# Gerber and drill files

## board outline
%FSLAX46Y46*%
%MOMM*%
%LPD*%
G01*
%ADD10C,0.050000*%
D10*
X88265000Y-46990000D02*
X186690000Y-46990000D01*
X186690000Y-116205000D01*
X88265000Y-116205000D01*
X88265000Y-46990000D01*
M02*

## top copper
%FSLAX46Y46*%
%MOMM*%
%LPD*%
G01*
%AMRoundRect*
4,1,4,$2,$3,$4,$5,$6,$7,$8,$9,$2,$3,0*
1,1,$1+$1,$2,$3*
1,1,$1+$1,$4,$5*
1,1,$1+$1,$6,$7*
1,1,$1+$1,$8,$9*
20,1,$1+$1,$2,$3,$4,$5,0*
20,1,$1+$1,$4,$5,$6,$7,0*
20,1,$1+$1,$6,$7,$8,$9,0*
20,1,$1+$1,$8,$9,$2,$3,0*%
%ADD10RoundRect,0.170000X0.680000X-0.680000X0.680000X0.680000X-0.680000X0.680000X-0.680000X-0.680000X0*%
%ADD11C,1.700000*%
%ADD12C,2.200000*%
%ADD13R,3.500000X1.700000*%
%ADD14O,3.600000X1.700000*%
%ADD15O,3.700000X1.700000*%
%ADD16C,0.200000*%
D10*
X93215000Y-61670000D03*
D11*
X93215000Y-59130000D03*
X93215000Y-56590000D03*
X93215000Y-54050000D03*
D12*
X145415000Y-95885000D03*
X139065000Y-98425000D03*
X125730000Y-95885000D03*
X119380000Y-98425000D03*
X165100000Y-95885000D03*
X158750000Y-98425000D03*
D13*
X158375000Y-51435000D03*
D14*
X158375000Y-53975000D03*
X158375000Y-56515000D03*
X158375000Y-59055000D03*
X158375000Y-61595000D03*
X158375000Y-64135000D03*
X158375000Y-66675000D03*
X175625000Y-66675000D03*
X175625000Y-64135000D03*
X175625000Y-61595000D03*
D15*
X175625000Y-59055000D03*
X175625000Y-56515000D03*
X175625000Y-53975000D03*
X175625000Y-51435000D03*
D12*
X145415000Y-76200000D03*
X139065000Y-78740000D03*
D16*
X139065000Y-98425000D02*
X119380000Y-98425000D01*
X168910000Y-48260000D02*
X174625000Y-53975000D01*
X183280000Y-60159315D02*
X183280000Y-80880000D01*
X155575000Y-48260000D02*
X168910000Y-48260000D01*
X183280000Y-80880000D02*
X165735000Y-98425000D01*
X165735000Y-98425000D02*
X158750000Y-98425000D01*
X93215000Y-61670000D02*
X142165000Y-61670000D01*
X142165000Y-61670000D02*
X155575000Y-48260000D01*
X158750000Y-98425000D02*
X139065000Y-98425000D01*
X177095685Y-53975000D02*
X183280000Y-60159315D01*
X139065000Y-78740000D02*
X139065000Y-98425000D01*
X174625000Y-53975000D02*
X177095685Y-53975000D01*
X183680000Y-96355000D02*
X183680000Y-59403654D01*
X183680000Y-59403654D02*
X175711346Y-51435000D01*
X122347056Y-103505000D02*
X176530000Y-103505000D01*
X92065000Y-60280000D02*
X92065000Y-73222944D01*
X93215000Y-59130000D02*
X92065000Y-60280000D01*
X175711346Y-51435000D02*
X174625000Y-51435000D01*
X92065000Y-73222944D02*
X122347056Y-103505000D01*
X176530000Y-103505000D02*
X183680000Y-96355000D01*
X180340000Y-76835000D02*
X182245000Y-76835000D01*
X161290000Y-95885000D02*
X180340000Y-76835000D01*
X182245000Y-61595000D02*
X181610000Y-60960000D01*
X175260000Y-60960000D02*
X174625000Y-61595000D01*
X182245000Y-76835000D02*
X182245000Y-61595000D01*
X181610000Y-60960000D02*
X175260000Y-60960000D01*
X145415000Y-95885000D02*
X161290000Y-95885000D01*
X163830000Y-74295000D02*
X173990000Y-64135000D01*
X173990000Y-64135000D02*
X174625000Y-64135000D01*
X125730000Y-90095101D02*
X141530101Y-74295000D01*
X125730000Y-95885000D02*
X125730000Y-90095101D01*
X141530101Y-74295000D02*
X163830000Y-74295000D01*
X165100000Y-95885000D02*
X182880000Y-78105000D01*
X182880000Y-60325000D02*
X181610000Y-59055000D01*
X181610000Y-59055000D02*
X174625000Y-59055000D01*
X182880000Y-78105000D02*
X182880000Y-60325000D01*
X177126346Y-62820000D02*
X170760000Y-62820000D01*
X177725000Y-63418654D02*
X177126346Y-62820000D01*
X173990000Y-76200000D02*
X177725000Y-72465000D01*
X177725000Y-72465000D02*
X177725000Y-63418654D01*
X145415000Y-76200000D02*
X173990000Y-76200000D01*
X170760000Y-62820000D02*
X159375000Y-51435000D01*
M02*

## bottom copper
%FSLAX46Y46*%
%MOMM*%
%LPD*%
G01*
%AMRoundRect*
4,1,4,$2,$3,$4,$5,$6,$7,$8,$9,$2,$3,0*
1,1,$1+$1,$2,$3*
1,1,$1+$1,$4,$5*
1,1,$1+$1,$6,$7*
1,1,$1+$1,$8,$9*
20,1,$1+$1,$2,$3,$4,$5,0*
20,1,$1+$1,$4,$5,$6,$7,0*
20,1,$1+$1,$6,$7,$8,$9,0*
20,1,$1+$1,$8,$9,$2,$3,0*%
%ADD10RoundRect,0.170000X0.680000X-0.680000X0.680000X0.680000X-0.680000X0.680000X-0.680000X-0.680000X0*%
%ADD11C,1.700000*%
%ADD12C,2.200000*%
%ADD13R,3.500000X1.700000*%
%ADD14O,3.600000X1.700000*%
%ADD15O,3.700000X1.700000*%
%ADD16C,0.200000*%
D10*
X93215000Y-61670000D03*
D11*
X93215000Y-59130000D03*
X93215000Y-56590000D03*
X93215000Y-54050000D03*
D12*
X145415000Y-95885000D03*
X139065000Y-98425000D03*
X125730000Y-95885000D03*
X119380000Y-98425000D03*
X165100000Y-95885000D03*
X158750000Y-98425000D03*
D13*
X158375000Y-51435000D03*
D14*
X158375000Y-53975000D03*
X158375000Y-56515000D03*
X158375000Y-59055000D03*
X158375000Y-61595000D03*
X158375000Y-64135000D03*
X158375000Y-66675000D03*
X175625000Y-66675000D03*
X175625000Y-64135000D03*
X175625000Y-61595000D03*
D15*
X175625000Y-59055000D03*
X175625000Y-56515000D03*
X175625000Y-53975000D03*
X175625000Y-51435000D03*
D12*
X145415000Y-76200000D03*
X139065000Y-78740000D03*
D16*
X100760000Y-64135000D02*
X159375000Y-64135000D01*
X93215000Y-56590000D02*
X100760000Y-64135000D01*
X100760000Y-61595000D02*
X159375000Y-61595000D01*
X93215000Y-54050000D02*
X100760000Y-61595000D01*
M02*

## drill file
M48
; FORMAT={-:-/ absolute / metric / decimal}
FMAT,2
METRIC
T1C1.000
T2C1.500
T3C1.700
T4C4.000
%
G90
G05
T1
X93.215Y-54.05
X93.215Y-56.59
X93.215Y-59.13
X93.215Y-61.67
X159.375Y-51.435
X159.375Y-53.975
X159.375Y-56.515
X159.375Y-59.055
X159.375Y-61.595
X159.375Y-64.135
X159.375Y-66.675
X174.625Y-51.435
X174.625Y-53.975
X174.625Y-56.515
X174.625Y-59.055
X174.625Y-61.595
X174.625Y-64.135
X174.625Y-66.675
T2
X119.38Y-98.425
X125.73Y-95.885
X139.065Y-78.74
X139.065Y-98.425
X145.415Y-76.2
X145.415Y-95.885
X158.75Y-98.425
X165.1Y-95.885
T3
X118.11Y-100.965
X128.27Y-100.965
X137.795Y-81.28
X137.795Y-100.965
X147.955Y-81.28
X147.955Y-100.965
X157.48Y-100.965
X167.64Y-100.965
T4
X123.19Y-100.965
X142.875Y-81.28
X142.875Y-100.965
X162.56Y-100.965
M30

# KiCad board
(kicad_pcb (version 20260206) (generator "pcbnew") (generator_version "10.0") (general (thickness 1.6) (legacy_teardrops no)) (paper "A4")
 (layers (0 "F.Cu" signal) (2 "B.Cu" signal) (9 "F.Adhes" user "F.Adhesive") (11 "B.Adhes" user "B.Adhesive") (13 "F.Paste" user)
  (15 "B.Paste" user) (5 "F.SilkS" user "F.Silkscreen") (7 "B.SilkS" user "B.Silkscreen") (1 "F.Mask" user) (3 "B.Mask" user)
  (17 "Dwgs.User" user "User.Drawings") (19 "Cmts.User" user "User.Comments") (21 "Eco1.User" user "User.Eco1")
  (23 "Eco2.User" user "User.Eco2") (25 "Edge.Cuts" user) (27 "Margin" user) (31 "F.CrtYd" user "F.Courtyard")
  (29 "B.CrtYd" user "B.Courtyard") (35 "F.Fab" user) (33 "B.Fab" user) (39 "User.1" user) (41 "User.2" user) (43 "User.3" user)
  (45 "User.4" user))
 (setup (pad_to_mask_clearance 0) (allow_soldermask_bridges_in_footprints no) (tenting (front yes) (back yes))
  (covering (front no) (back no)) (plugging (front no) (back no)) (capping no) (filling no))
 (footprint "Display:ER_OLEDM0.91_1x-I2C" (layer "F.Cu") (at 93.215 61.67 90)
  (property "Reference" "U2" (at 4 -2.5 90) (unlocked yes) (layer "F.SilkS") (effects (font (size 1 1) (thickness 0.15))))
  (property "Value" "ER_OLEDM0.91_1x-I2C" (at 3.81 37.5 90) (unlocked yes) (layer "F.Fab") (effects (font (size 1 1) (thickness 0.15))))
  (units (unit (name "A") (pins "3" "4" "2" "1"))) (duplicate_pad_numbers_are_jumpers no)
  (pad "1" thru_hole roundrect (at 0 0 90) (size 1.7 1.7) (drill 1) (layers "*.Cu" "*.Mask") (remove_unused_layers no)
   (roundrect_rratio 0.1) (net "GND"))
  (pad "2" thru_hole circle (at 2.54 0 90) (size 1.7 1.7) (drill 1) (layers "*.Cu" "*.Mask") (remove_unused_layers no) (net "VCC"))
  (pad "3" thru_hole circle (at 5.08 0 90) (size 1.7 1.7) (drill 1) (layers "*.Cu" "*.Mask") (remove_unused_layers no)
   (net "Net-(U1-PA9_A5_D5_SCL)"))
  (pad "4" thru_hole circle (at 7.62 0 90) (size 1.7 1.7) (drill 1) (layers "*.Cu" "*.Mask") (remove_unused_layers no)
   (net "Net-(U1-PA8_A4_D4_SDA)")))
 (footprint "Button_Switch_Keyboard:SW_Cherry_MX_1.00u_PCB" (layer "F.Cu") (at 145.415 95.885)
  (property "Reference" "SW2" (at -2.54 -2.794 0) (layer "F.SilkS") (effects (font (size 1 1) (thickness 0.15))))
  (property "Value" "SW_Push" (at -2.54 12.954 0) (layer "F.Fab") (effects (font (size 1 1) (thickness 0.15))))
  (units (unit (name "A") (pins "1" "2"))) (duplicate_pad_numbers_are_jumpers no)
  (pad "" np_thru_hole circle (at -7.62 5.08) (size 1.7 1.7) (drill 1.7) (layers "*.Cu" "*.Mask"))
  (pad "" np_thru_hole circle (at -2.54 5.08) (size 4 4) (drill 4) (layers "*.Cu" "*.Mask"))
  (pad "" np_thru_hole circle (at 2.54 5.08) (size 1.7 1.7) (drill 1.7) (layers "*.Cu" "*.Mask"))
  (pad "1" thru_hole circle (at 0 0) (size 2.2 2.2) (drill 1.5) (layers "*.Cu" "*.Mask") (remove_unused_layers no)
   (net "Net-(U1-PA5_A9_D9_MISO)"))
  (pad "2" thru_hole circle (at -6.35 2.54) (size 2.2 2.2) (drill 1.5) (layers "*.Cu" "*.Mask") (remove_unused_layers no) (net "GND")))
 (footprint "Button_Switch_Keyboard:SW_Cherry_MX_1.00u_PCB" (layer "F.Cu") (at 125.73 95.885)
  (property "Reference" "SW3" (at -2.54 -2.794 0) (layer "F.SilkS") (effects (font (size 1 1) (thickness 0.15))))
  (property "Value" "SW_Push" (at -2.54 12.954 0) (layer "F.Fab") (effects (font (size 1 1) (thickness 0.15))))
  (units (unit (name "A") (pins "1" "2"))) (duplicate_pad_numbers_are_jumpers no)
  (pad "" np_thru_hole circle (at -7.62 5.08) (size 1.7 1.7) (drill 1.7) (layers "*.Cu" "*.Mask"))
  (pad "" np_thru_hole circle (at -2.54 5.08) (size 4 4) (drill 4) (layers "*.Cu" "*.Mask"))
  (pad "" np_thru_hole circle (at 2.54 5.08) (size 1.7 1.7) (drill 1.7) (layers "*.Cu" "*.Mask"))
  (pad "1" thru_hole circle (at 0 0) (size 2.2 2.2) (drill 1.5) (layers "*.Cu" "*.Mask") (remove_unused_layers no)
   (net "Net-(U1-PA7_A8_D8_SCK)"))
  (pad "2" thru_hole circle (at -6.35 2.54) (size 2.2 2.2) (drill 1.5) (layers "*.Cu" "*.Mask") (remove_unused_layers no) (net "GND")))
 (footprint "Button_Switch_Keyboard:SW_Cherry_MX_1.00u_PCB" (layer "F.Cu") (at 165.1 95.885)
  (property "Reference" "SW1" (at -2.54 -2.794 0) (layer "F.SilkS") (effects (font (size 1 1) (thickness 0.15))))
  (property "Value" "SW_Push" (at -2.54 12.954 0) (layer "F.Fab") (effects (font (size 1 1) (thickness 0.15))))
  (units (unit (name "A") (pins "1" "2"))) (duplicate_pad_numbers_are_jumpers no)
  (pad "" np_thru_hole circle (at -7.62 5.08) (size 1.7 1.7) (drill 1.7) (layers "*.Cu" "*.Mask"))
  (pad "" np_thru_hole circle (at -2.54 5.08) (size 4 4) (drill 4) (layers "*.Cu" "*.Mask"))
  (pad "" np_thru_hole circle (at 2.54 5.08) (size 1.7 1.7) (drill 1.7) (layers "*.Cu" "*.Mask"))
  (pad "1" thru_hole circle (at 0 0) (size 2.2 2.2) (drill 1.5) (layers "*.Cu" "*.Mask") (remove_unused_layers no)
   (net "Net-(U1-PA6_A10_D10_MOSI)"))
  (pad "2" thru_hole circle (at -6.35 2.54) (size 2.2 2.2) (drill 1.5) (layers "*.Cu" "*.Mask") (remove_unused_layers no) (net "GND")))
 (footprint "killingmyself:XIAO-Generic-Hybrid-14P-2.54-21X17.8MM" (layer "F.Cu") (at 167 59.055)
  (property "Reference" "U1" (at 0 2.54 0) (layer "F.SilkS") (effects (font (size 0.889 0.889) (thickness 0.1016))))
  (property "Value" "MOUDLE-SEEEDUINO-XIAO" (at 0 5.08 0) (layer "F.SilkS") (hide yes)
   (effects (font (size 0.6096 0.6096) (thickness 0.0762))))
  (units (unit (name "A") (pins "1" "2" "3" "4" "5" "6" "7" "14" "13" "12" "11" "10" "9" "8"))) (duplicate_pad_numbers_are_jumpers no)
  (pad "1" thru_hole rect (at -7.625 -7.62) (size 3.5 1.7) (drill 1 (offset -1 0)) (layers "*.Cu" "*.Mask") (remove_unused_layers no)
   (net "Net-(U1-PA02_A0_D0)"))
  (pad "2" thru_hole oval (at -7.625 -5.08) (size 3.6 1.7) (drill 1 (offset -1 0)) (layers "*.Cu" "*.Mask") (remove_unused_layers no)
   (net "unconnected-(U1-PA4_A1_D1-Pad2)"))
  (pad "3" thru_hole oval (at -7.625 -2.54) (size 3.6 1.7) (drill 1 (offset -1 0)) (layers "*.Cu" "*.Mask") (remove_unused_layers no)
   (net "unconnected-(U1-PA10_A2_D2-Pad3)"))
  (pad "4" thru_hole oval (at -7.625 0) (size 3.6 1.7) (drill 1 (offset -1 0)) (layers "*.Cu" "*.Mask") (remove_unused_layers no)
   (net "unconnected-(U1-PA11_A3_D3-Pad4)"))
  (pad "5" thru_hole oval (at -7.625 2.54) (size 3.6 1.7) (drill 1 (offset -1 0)) (layers "*.Cu" "*.Mask") (remove_unused_layers no)
   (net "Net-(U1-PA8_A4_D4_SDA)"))
  (pad "6" thru_hole oval (at -7.625 5.08 180) (size 3.6 1.7) (drill 1 (offset 1 0)) (layers "*.Cu" "*.Mask") (remove_unused_layers no)
   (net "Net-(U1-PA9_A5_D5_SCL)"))
  (pad "7" thru_hole oval (at -7.625 7.62) (size 3.6 1.7) (drill 1 (offset -1 0)) (layers "*.Cu" "*.Mask") (remove_unused_layers no)
   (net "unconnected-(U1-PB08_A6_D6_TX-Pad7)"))
  (pad "8" thru_hole oval (at 7.625 7.62) (size 3.6 1.7) (drill 1 (offset 1 0)) (layers "*.Cu" "*.Mask") (remove_unused_layers no)
   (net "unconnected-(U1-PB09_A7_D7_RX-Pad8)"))
  (pad "9" thru_hole oval (at 7.625 5.08) (size 3.6 1.7) (drill 1 (offset 1 0)) (layers "*.Cu" "*.Mask") (remove_unused_layers no)
   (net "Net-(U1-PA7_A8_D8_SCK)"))
  (pad "10" thru_hole oval (at 7.625 2.54) (size 3.6 1.7) (drill 1 (offset 1 0)) (layers "*.Cu" "*.Mask") (remove_unused_layers no)
   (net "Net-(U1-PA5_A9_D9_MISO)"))
  (pad "11" thru_hole oval (at 7.625 0) (size 3.7 1.7) (drill 1 (offset 1 0)) (layers "*.Cu" "*.Mask") (remove_unused_layers no)
   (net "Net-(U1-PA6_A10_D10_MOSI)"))
  (pad "12" thru_hole oval (at 7.625 -2.54) (size 3.7 1.7) (drill 1 (offset 1 0)) (layers "*.Cu" "*.Mask") (remove_unused_layers no)
   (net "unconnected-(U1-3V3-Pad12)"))
  (pad "13" thru_hole oval (at 7.625 -5.08) (size 3.7 1.7) (drill 1 (offset 1 0)) (layers "*.Cu" "*.Mask") (remove_unused_layers no)
   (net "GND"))
  (pad "14" thru_hole oval (at 7.625 -7.62) (size 3.7 1.7) (drill 1 (offset 1 0)) (layers "*.Cu" "*.Mask") (remove_unused_layers no)
   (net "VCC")))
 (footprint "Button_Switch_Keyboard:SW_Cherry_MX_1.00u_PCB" (layer "F.Cu") (at 145.415 76.2)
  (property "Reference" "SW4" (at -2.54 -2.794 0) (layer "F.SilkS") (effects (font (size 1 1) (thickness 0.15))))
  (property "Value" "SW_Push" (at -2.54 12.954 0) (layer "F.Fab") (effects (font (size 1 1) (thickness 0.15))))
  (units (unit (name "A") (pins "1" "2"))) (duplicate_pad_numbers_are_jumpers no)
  (pad "" np_thru_hole circle (at -7.62 5.08) (size 1.7 1.7) (drill 1.7) (layers "*.Cu" "*.Mask"))
  (pad "" np_thru_hole circle (at -2.54 5.08) (size 4 4) (drill 4) (layers "*.Cu" "*.Mask"))
  (pad "" np_thru_hole circle (at 2.54 5.08) (size 1.7 1.7) (drill 1.7) (layers "*.Cu" "*.Mask"))
  (pad "1" thru_hole circle (at 0 0) (size 2.2 2.2) (drill 1.5) (layers "*.Cu" "*.Mask") (remove_unused_layers no)
   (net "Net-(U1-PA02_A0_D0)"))
  (pad "2" thru_hole circle (at -6.35 2.54) (size 2.2 2.2) (drill 1.5) (layers "*.Cu" "*.Mask") (remove_unused_layers no) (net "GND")))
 (gr_rect (start 88.265 46.99) (end 186.69 116.205) (stroke (width 0.05) (type default)) (fill no) (layer "Edge.Cuts"))
 (segment (start 139.065 98.425) (end 119.38 98.425) (width 0.2) (layer "F.Cu") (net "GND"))
 (segment (start 168.91 48.26) (end 174.625 53.975) (width 0.2) (layer "F.Cu") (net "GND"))
 (segment (start 183.28 60.159315) (end 183.28 80.88) (width 0.2) (layer "F.Cu") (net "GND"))
 (segment (start 155.575 48.26) (end 168.91 48.26) (width 0.2) (layer "F.Cu") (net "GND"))
 (segment (start 183.28 80.88) (end 165.735 98.425) (width 0.2) (layer "F.Cu") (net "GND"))
 (segment (start 165.735 98.425) (end 158.75 98.425) (width 0.2) (layer "F.Cu") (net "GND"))
 (segment (start 93.215 61.67) (end 142.165 61.67) (width 0.2) (layer "F.Cu") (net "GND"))
 (segment (start 142.165 61.67) (end 155.575 48.26) (width 0.2) (layer "F.Cu") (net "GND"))
 (segment (start 158.75 98.425) (end 139.065 98.425) (width 0.2) (layer "F.Cu") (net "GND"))
 (segment (start 177.095685 53.975) (end 183.28 60.159315) (width 0.2) (layer "F.Cu") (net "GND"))
 (segment (start 139.065 78.74) (end 139.065 98.425) (width 0.2) (layer "F.Cu") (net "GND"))
 (segment (start 174.625 53.975) (end 177.095685 53.975) (width 0.2) (layer "F.Cu") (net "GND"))
 (segment (start 183.68 96.355) (end 183.68 59.403654) (width 0.2) (layer "F.Cu") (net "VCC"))
 (segment (start 183.68 59.403654) (end 175.711346 51.435) (width 0.2) (layer "F.Cu") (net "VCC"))
 (segment (start 122.347056 103.505) (end 176.53 103.505) (width 0.2) (layer "F.Cu") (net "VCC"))
 (segment (start 92.065 60.28) (end 92.065 73.222944) (width 0.2) (layer "F.Cu") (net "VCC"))
 (segment (start 93.215 59.13) (end 92.065 60.28) (width 0.2) (layer "F.Cu") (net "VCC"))
 (segment (start 175.711346 51.435) (end 174.625 51.435) (width 0.2) (layer "F.Cu") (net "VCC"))
 (segment (start 92.065 73.222944) (end 122.347056 103.505) (width 0.2) (layer "F.Cu") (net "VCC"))
 (segment (start 176.53 103.505) (end 183.68 96.355) (width 0.2) (layer "F.Cu") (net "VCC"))
 (segment (start 100.76 64.135) (end 159.375 64.135) (width 0.2) (layer "B.Cu") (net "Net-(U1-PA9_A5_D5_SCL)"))
 (segment (start 93.215 56.59) (end 100.76 64.135) (width 0.2) (layer "B.Cu") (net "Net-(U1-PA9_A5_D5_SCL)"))
 (segment (start 100.76 61.595) (end 159.375 61.595) (width 0.2) (layer "B.Cu") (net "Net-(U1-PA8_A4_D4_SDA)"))
 (segment (start 93.215 54.05) (end 100.76 61.595) (width 0.2) (layer "B.Cu") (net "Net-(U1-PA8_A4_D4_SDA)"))
 (segment (start 180.34 76.835) (end 182.245 76.835) (width 0.2) (layer "F.Cu") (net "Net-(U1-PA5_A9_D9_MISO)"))
 (segment (start 161.29 95.885) (end 180.34 76.835) (width 0.2) (layer "F.Cu") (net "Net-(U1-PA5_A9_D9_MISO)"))
 (segment (start 182.245 61.595) (end 181.61 60.96) (width 0.2) (layer "F.Cu") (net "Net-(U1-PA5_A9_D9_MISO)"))
 (segment (start 175.26 60.96) (end 174.625 61.595) (width 0.2) (layer "F.Cu") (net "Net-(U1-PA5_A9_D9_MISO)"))
 (segment (start 182.245 76.835) (end 182.245 61.595) (width 0.2) (layer "F.Cu") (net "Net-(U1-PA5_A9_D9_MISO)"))
 (segment (start 181.61 60.96) (end 175.26 60.96) (width 0.2) (layer "F.Cu") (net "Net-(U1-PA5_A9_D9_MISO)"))
 (segment (start 145.415 95.885) (end 161.29 95.885) (width 0.2) (layer "F.Cu") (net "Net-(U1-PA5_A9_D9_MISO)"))
 (segment (start 163.83 74.295) (end 173.99 64.135) (width 0.2) (layer "F.Cu") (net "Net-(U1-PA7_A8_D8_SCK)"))
 (segment (start 173.99 64.135) (end 174.625 64.135) (width 0.2) (layer "F.Cu") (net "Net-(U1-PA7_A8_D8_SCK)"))
 (segment (start 125.73 90.095101) (end 141.530101 74.295) (width 0.2) (layer "F.Cu") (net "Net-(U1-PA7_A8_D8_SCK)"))
 (segment (start 125.73 95.885) (end 125.73 90.095101) (width 0.2) (layer "F.Cu") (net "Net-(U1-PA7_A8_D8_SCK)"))
 (segment (start 141.530101 74.295) (end 163.83 74.295) (width 0.2) (layer "F.Cu") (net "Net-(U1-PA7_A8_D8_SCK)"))
 (segment (start 165.1 95.885) (end 182.88 78.105) (width 0.2) (layer "F.Cu") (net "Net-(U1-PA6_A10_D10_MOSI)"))
 (segment (start 182.88 60.325) (end 181.61 59.055) (width 0.2) (layer "F.Cu") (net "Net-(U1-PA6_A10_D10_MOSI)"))
 (segment (start 181.61 59.055) (end 174.625 59.055) (width 0.2) (layer "F.Cu") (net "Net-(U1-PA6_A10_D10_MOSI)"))
 (segment (start 182.88 78.105) (end 182.88 60.325) (width 0.2) (layer "F.Cu") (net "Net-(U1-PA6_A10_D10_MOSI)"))
 (segment (start 177.126346 62.82) (end 170.76 62.82) (width 0.2) (layer "F.Cu") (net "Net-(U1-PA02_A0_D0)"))
 (segment (start 177.725 63.418654) (end 177.126346 62.82) (width 0.2) (layer "F.Cu") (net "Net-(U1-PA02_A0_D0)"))
 (segment (start 173.99 76.2) (end 177.725 72.465) (width 0.2) (layer "F.Cu") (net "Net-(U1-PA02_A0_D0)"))
 (segment (start 177.725 72.465) (end 177.725 63.418654) (width 0.2) (layer "F.Cu") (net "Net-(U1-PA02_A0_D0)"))
 (segment (start 145.415 76.2) (end 173.99 76.2) (width 0.2) (layer "F.Cu") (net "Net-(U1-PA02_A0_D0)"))
 (segment (start 170.76 62.82) (end 159.375 51.435) (width 0.2) (layer "F.Cu") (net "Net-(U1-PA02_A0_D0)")))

